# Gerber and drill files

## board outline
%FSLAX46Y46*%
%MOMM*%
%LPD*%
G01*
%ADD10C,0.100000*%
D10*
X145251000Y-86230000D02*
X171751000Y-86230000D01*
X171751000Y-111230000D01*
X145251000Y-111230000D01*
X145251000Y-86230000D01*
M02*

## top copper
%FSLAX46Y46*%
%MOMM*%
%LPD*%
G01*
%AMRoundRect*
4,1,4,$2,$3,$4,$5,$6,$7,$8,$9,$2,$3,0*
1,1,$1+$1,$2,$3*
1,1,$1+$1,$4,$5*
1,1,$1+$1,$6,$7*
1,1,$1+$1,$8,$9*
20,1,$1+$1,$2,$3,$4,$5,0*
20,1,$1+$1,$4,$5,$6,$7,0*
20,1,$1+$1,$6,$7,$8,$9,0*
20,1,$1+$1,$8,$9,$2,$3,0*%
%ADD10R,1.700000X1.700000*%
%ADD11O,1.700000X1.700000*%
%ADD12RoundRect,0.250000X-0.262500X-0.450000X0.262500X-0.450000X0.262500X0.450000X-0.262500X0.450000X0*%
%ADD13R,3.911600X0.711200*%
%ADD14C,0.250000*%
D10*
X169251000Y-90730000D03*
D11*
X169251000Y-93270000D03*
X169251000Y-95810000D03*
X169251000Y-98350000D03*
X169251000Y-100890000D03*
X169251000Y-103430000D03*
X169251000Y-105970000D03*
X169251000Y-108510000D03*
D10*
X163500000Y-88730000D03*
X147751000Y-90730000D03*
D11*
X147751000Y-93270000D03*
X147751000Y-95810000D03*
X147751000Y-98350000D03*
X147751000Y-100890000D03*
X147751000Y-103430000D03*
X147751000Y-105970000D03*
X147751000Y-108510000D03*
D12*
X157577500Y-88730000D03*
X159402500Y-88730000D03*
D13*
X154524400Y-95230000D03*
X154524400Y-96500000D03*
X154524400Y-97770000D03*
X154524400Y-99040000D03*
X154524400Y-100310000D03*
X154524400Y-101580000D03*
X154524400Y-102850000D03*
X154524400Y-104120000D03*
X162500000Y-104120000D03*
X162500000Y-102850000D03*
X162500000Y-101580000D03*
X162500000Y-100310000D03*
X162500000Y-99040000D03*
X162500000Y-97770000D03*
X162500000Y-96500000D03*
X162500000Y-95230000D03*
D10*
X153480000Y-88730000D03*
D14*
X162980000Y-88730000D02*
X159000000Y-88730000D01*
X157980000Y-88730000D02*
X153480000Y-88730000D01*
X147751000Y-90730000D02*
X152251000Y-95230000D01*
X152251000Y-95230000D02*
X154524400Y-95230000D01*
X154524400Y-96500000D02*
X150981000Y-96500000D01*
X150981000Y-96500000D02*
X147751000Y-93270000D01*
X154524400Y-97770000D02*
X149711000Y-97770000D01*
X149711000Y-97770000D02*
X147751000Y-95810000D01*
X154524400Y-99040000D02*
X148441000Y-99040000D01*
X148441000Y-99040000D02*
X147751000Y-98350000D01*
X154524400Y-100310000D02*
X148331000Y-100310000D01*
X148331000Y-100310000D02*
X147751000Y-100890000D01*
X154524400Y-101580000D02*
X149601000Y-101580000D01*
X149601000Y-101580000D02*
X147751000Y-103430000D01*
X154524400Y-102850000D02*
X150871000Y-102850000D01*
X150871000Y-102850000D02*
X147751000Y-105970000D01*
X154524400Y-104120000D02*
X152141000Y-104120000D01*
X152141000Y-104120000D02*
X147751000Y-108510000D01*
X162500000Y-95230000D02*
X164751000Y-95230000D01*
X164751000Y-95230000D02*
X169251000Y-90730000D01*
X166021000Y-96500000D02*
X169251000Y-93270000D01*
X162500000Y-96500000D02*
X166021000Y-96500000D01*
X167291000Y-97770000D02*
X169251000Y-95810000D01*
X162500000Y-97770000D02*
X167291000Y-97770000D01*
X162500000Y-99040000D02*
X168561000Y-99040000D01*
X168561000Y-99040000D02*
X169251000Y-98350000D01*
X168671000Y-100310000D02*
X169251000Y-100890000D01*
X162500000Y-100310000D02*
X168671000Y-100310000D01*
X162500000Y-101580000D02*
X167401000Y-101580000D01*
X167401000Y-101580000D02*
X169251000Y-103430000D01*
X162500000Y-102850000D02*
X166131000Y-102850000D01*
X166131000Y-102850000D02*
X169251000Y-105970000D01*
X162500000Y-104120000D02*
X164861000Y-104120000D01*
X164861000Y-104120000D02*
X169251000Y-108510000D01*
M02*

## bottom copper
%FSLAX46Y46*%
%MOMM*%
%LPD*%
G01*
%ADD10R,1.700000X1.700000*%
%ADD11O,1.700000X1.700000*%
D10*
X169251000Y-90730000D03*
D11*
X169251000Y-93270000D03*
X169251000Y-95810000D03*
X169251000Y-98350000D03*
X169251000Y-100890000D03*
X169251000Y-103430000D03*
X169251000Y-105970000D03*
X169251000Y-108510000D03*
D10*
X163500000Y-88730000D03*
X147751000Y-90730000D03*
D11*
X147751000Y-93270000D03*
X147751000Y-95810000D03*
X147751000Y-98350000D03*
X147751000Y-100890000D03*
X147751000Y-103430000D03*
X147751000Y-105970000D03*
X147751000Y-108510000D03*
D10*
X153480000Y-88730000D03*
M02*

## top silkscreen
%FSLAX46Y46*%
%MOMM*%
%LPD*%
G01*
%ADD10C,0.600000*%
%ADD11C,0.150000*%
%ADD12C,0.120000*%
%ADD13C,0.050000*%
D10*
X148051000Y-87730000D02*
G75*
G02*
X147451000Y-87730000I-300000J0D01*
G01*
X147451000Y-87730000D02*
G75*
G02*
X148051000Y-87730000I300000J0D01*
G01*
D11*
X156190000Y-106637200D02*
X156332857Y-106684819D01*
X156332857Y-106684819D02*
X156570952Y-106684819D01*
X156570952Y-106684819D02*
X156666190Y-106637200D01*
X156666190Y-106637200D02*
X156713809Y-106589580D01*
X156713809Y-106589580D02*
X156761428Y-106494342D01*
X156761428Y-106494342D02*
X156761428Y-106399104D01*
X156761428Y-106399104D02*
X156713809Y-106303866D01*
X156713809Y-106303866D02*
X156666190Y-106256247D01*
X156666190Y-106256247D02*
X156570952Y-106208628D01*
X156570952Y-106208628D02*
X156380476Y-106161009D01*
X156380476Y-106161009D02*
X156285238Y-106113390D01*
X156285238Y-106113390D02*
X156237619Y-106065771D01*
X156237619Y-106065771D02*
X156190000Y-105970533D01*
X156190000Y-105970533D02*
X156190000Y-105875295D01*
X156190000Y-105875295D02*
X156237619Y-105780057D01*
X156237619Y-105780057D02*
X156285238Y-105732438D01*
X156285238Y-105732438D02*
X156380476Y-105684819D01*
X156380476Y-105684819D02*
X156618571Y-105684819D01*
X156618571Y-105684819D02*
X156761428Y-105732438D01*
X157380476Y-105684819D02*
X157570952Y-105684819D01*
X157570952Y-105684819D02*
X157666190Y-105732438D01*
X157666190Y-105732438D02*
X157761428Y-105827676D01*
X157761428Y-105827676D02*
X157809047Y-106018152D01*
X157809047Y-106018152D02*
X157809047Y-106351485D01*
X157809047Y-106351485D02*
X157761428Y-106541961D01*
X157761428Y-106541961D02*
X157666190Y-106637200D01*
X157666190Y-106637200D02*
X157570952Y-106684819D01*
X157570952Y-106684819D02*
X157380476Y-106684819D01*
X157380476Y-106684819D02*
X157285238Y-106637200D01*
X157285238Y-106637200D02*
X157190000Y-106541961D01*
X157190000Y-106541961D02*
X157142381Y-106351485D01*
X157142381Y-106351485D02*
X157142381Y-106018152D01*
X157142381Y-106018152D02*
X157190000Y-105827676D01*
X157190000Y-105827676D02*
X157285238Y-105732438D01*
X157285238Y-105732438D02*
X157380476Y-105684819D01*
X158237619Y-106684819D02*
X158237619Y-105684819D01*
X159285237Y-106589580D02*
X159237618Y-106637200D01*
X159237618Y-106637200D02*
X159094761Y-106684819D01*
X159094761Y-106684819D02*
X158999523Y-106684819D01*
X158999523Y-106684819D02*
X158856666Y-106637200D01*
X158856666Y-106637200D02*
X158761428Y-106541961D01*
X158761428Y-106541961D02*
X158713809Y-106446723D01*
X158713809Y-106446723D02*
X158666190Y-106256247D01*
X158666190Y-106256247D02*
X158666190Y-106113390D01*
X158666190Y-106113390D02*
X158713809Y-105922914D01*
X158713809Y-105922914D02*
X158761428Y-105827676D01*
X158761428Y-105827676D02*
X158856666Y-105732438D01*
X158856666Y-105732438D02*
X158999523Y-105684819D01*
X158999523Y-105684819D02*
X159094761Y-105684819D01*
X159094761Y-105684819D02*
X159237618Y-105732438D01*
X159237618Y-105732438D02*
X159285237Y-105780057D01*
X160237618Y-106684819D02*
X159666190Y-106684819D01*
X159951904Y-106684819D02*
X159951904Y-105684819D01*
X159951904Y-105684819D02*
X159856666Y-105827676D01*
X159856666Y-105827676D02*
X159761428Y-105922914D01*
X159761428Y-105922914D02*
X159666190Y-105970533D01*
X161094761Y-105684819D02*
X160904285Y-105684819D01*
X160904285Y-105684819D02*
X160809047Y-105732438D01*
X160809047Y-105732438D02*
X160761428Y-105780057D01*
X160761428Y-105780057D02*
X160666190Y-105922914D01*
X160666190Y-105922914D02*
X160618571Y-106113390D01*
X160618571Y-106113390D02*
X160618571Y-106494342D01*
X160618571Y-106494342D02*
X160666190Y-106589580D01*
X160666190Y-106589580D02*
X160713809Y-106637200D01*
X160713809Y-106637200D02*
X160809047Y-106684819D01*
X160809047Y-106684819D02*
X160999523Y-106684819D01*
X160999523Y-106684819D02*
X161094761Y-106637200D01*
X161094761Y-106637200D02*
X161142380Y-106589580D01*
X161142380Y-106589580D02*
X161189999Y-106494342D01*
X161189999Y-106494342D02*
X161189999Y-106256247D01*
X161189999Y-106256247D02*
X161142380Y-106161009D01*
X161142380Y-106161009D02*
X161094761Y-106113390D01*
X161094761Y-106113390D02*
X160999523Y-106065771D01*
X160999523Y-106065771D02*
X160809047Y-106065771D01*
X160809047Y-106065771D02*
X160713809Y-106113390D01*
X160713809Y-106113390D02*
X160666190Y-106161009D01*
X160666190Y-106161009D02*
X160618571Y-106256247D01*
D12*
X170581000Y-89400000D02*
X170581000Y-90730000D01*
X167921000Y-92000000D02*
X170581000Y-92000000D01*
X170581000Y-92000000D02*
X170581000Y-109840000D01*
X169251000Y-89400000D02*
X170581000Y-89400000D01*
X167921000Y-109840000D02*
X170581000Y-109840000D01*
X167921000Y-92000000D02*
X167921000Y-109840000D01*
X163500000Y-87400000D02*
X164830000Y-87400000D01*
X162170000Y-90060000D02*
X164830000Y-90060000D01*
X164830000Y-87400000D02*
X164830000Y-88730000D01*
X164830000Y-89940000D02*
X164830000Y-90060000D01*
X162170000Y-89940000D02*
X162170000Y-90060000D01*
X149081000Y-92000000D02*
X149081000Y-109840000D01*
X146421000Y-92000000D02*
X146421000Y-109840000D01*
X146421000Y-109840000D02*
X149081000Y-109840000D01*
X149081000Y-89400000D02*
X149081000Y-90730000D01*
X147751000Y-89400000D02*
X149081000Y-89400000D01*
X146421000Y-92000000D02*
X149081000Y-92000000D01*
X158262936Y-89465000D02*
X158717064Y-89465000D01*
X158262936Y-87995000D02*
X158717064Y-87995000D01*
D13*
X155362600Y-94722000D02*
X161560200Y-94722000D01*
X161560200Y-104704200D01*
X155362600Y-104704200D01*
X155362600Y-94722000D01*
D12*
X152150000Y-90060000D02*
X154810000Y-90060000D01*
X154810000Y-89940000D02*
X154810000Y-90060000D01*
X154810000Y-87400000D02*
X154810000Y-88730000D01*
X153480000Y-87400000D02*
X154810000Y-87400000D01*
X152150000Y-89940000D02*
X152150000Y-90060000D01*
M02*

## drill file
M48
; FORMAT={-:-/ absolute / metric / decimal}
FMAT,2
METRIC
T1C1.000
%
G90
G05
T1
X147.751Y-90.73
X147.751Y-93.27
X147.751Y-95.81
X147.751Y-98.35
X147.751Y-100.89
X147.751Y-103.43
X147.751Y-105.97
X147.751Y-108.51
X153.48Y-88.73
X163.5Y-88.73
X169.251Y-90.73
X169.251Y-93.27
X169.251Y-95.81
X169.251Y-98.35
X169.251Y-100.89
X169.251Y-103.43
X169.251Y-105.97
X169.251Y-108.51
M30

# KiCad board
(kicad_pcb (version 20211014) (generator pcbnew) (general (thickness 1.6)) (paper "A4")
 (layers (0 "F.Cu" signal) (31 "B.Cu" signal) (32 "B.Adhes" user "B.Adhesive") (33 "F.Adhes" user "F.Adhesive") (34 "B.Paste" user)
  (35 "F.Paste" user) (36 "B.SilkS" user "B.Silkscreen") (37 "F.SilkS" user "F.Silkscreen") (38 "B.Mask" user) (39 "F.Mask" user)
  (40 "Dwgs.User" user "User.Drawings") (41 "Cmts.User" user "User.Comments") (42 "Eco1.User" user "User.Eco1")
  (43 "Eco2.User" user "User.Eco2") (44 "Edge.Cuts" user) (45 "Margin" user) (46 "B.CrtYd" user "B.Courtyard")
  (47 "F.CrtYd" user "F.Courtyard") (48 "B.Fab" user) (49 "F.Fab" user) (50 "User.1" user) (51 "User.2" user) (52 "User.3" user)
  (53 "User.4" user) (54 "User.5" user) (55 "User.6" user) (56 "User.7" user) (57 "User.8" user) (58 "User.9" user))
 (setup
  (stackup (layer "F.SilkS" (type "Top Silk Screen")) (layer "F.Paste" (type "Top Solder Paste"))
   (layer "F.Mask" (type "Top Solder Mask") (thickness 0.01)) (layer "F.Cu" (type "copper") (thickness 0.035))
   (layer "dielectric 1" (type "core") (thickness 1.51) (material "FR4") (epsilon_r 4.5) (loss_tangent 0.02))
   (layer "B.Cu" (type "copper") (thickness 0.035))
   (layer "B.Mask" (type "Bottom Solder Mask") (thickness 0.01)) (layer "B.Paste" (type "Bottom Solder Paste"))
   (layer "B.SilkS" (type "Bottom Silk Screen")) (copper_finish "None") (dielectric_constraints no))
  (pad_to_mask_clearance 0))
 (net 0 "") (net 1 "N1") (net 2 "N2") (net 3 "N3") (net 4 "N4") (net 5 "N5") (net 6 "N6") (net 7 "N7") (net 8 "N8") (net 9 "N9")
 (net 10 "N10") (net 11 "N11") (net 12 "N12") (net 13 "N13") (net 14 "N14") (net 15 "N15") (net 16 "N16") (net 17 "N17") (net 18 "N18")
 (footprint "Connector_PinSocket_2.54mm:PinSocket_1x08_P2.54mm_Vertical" (layer "F.Cu") (at 169.251 90.73)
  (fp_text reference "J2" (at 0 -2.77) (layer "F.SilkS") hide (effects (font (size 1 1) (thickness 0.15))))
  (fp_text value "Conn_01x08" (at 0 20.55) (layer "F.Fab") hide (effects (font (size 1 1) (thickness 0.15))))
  (fp_line (start 1.33 -1.33) (end 1.33 0) (layer "F.SilkS") (width 0.12))
  (fp_line (start -1.33 1.27) (end 1.33 1.27) (layer "F.SilkS") (width 0.12))
  (fp_line (start 1.33 1.27) (end 1.33 19.11) (layer "F.SilkS") (width 0.12))
  (fp_line (start 0 -1.33) (end 1.33 -1.33) (layer "F.SilkS") (width 0.12))
  (fp_line (start -1.33 19.11) (end 1.33 19.11) (layer "F.SilkS") (width 0.12))
  (fp_line (start -1.33 1.27) (end -1.33 19.11) (layer "F.SilkS") (width 0.12))
  (pad "1" thru_hole rect (at 0 0) (size 1.7 1.7) (drill 1) (layers *.Cu *.Mask) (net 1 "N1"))
  (pad "2" thru_hole oval (at 0 2.54) (size 1.7 1.7) (drill 1) (layers *.Cu *.Mask) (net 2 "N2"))
  (pad "3" thru_hole oval (at 0 5.08) (size 1.7 1.7) (drill 1) (layers *.Cu *.Mask) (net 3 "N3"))
  (pad "4" thru_hole oval (at 0 7.62) (size 1.7 1.7) (drill 1) (layers *.Cu *.Mask) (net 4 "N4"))
  (pad "5" thru_hole oval (at 0 10.16) (size 1.7 1.7) (drill 1) (layers *.Cu *.Mask) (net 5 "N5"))
  (pad "6" thru_hole oval (at 0 12.7) (size 1.7 1.7) (drill 1) (layers *.Cu *.Mask) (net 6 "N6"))
  (pad "7" thru_hole oval (at 0 15.24) (size 1.7 1.7) (drill 1) (layers *.Cu *.Mask) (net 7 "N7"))
  (pad "8" thru_hole oval (at 0 17.78) (size 1.7 1.7) (drill 1) (layers *.Cu *.Mask) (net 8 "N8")))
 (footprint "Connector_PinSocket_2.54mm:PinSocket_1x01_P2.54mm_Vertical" (layer "F.Cu") (at 163.5 88.73)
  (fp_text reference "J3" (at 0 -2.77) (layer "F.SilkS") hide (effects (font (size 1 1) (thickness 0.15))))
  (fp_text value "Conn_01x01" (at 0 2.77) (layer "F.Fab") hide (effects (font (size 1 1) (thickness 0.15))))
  (fp_line (start 0 -1.33) (end 1.33 -1.33) (layer "F.SilkS") (width 0.12))
  (fp_line (start -1.33 1.33) (end 1.33 1.33) (layer "F.SilkS") (width 0.12))
  (fp_line (start 1.33 -1.33) (end 1.33 0) (layer "F.SilkS") (width 0.12))
  (fp_line (start 1.33 1.21) (end 1.33 1.33) (layer "F.SilkS") (width 0.12))
  (fp_line (start -1.33 1.21) (end -1.33 1.33) (layer "F.SilkS") (width 0.12))
  (pad "1" thru_hole rect (at 0 0) (size 1.7 1.7) (drill 1) (layers *.Cu *.Mask) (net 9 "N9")))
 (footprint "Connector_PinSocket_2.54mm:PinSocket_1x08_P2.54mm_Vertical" (layer "F.Cu") (at 147.751 90.73)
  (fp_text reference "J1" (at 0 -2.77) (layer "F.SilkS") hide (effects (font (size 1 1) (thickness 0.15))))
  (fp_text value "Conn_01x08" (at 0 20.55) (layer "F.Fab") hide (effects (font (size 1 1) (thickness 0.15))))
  (fp_line (start 1.33 1.27) (end 1.33 19.11) (layer "F.SilkS") (width 0.12))
  (fp_line (start -1.33 1.27) (end -1.33 19.11) (layer "F.SilkS") (width 0.12))
  (fp_line (start -1.33 19.11) (end 1.33 19.11) (layer "F.SilkS") (width 0.12))
  (fp_line (start 1.33 -1.33) (end 1.33 0) (layer "F.SilkS") (width 0.12))
  (fp_line (start 0 -1.33) (end 1.33 -1.33) (layer "F.SilkS") (width 0.12))
  (fp_line (start -1.33 1.27) (end 1.33 1.27) (layer "F.SilkS") (width 0.12))
  (pad "1" thru_hole rect (at 0 0) (size 1.7 1.7) (drill 1) (layers *.Cu *.Mask) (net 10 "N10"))
  (pad "2" thru_hole oval (at 0 2.54) (size 1.7 1.7) (drill 1) (layers *.Cu *.Mask) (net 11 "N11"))
  (pad "3" thru_hole oval (at 0 5.08) (size 1.7 1.7) (drill 1) (layers *.Cu *.Mask) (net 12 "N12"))
  (pad "4" thru_hole oval (at 0 7.62) (size 1.7 1.7) (drill 1) (layers *.Cu *.Mask) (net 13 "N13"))
  (pad "5" thru_hole oval (at 0 10.16) (size 1.7 1.7) (drill 1) (layers *.Cu *.Mask) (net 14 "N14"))
  (pad "6" thru_hole oval (at 0 12.7) (size 1.7 1.7) (drill 1) (layers *.Cu *.Mask) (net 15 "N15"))
  (pad "7" thru_hole oval (at 0 15.24) (size 1.7 1.7) (drill 1) (layers *.Cu *.Mask) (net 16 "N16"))
  (pad "8" thru_hole oval (at 0 17.78) (size 1.7 1.7) (drill 1) (layers *.Cu *.Mask) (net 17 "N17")))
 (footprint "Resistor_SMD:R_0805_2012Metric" (layer "F.Cu") (at 158.49 88.73)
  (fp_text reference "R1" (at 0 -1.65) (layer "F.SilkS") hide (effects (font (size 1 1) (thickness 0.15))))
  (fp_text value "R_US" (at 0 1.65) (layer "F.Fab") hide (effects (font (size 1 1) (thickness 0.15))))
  (fp_line (start -0.227064 0.735) (end 0.227064 0.735) (layer "F.SilkS") (width 0.12))
  (fp_line (start -0.227064 -0.735) (end 0.227064 -0.735) (layer "F.SilkS") (width 0.12))
  (pad "1" smd roundrect (at -0.9125 0) (size 1.025 1.4) (layers "F.Cu" "F.Paste" "F.Mask") (roundrect_rratio 0.243902) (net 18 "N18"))
  (pad "2" smd roundrect (at 0.9125 0) (size 1.025 1.4) (layers "F.Cu" "F.Paste" "F.Mask") (roundrect_rratio 0.243902) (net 9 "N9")))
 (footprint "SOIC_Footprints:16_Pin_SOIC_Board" (layer "F.Cu") (at 158.69 99.548)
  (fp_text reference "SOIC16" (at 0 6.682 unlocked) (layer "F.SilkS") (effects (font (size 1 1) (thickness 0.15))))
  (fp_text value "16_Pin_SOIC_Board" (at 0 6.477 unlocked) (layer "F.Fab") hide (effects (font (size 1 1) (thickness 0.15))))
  (fp_rect (start -3.3274 -4.826) (end 2.8702 5.1562) (layer "F.SilkS") (width 0.05) (fill none))
  (pad "1" smd rect (at -4.1656 -4.318) (size 3.9116 0.7112) (layers "F.Cu" "F.Paste" "F.Mask") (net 10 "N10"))
  (pad "2" smd rect (at -4.1656 -3.048) (size 3.9116 0.7112) (layers "F.Cu" "F.Paste" "F.Mask") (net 11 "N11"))
  (pad "3" smd rect (at -4.1656 -1.778) (size 3.9116 0.7112) (layers "F.Cu" "F.Paste" "F.Mask") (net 12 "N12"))
  (pad "4" smd rect (at -4.1656 -0.508) (size 3.9116 0.7112) (layers "F.Cu" "F.Paste" "F.Mask") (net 13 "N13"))
  (pad "5" smd rect (at -4.1656 0.762) (size 3.9116 0.7112) (layers "F.Cu" "F.Paste" "F.Mask") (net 14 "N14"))
  (pad "6" smd rect (at -4.1656 2.032) (size 3.9116 0.7112) (layers "F.Cu" "F.Paste" "F.Mask") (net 15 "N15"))
  (pad "7" smd rect (at -4.1656 3.302) (size 3.9116 0.7112) (layers "F.Cu" "F.Paste" "F.Mask") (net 16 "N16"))
  (pad "8" smd rect (at -4.1656 4.572) (size 3.9116 0.7112) (layers "F.Cu" "F.Paste" "F.Mask") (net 17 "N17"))
  (pad "9" smd rect (at 3.81 4.572) (size 3.9116 0.7112) (layers "F.Cu" "F.Paste" "F.Mask") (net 8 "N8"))
  (pad "10" smd rect (at 3.81 3.302) (size 3.9116 0.7112) (layers "F.Cu" "F.Paste" "F.Mask") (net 7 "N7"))
  (pad "11" smd rect (at 3.81 2.032) (size 3.9116 0.7112) (layers "F.Cu" "F.Paste" "F.Mask") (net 6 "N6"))
  (pad "12" smd rect (at 3.81 0.762) (size 3.9116 0.7112) (layers "F.Cu" "F.Paste" "F.Mask") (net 5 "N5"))
  (pad "13" smd rect (at 3.81 -0.508) (size 3.9116 0.7112) (layers "F.Cu" "F.Paste" "F.Mask") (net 4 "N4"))
  (pad "14" smd rect (at 3.81 -1.778) (size 3.9116 0.7112) (layers "F.Cu" "F.Paste" "F.Mask") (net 3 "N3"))
  (pad "15" smd rect (at 3.81 -3.048) (size 3.9116 0.7112) (layers "F.Cu" "F.Paste" "F.Mask") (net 2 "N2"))
  (pad "16" smd rect (at 3.81 -4.318) (size 3.9116 0.7112) (layers "F.Cu" "F.Paste" "F.Mask") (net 1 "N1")))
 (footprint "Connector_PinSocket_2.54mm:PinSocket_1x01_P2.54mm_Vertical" (layer "F.Cu") (at 153.48 88.73)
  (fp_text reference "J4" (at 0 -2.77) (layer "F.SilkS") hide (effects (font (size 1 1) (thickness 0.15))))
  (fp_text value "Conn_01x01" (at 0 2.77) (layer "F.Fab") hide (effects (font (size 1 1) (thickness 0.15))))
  (fp_line (start -1.33 1.33) (end 1.33 1.33) (layer "F.SilkS") (width 0.12))
  (fp_line (start 1.33 1.21) (end 1.33 1.33) (layer "F.SilkS") (width 0.12))
  (fp_line (start 1.33 -1.33) (end 1.33 0) (layer "F.SilkS") (width 0.12))
  (fp_line (start 0 -1.33) (end 1.33 -1.33) (layer "F.SilkS") (width 0.12))
  (fp_line (start -1.33 1.21) (end -1.33 1.33) (layer "F.SilkS") (width 0.12))
  (pad "1" thru_hole rect (at 0 0) (size 1.7 1.7) (drill 1) (layers *.Cu *.Mask) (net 18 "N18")))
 (gr_circle (center 147.751 87.73) (end 148.251 87.73) (layer "F.SilkS") (width 0.2) (fill solid))
 (gr_rect (start 145.251 86.23) (end 171.751 111.23) (layer "Edge.Cuts") (width 0.1) (fill none))
 (segment (start 162.98 88.73) (end 159 88.73) (width 0.25) (layer "F.Cu") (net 9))
 (segment (start 157.98 88.73) (end 153.48 88.73) (width 0.25) (layer "F.Cu") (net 18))
 (segment (start 147.751 90.73) (end 152.251 95.23) (width 0.25) (layer "F.Cu") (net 10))
 (segment (start 152.251 95.23) (end 154.5244 95.23) (width 0.25) (layer "F.Cu") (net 10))
 (segment (start 154.5244 96.5) (end 150.981 96.5) (width 0.25) (layer "F.Cu") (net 11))
 (segment (start 150.981 96.5) (end 147.751 93.27) (width 0.25) (layer "F.Cu") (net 11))
 (segment (start 154.5244 97.77) (end 149.711 97.77) (width 0.25) (layer "F.Cu") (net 12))
 (segment (start 149.711 97.77) (end 147.751 95.81) (width 0.25) (layer "F.Cu") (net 12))
 (segment (start 154.5244 99.04) (end 148.441 99.04) (width 0.25) (layer "F.Cu") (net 13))
 (segment (start 148.441 99.04) (end 147.751 98.35) (width 0.25) (layer "F.Cu") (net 13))
 (segment (start 154.5244 100.31) (end 148.331 100.31) (width 0.25) (layer "F.Cu") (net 14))
 (segment (start 148.331 100.31) (end 147.751 100.89) (width 0.25) (layer "F.Cu") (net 14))
 (segment (start 154.5244 101.58) (end 149.601 101.58) (width 0.25) (layer "F.Cu") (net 15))
 (segment (start 149.601 101.58) (end 147.751 103.43) (width 0.25) (layer "F.Cu") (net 15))
 (segment (start 154.5244 102.85) (end 150.871 102.85) (width 0.25) (layer "F.Cu") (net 16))
 (segment (start 150.871 102.85) (end 147.751 105.97) (width 0.25) (layer "F.Cu") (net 16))
 (segment (start 154.5244 104.12) (end 152.141 104.12) (width 0.25) (layer "F.Cu") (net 17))
 (segment (start 152.141 104.12) (end 147.751 108.51) (width 0.25) (layer "F.Cu") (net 17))
 (segment (start 162.5 95.23) (end 164.751 95.23) (width 0.25) (layer "F.Cu") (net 1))
 (segment (start 164.751 95.23) (end 169.251 90.73) (width 0.25) (layer "F.Cu") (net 1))
 (segment (start 166.021 96.5) (end 169.251 93.27) (width 0.25) (layer "F.Cu") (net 2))
 (segment (start 162.5 96.5) (end 166.021 96.5) (width 0.25) (layer "F.Cu") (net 2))
 (segment (start 167.291 97.77) (end 169.251 95.81) (width 0.25) (layer "F.Cu") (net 3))
 (segment (start 162.5 97.77) (end 167.291 97.77) (width 0.25) (layer "F.Cu") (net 3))
 (segment (start 162.5 99.04) (end 168.561 99.04) (width 0.25) (layer "F.Cu") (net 4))
 (segment (start 168.561 99.04) (end 169.251 98.35) (width 0.25) (layer "F.Cu") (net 4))
 (segment (start 168.671 100.31) (end 169.251 100.89) (width 0.25) (layer "F.Cu") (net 5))
 (segment (start 162.5 100.31) (end 168.671 100.31) (width 0.25) (layer "F.Cu") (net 5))
 (segment (start 162.5 101.58) (end 167.401 101.58) (width 0.25) (layer "F.Cu") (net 6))
 (segment (start 167.401 101.58) (end 169.251 103.43) (width 0.25) (layer "F.Cu") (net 6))
 (segment (start 162.5 102.85) (end 166.131 102.85) (width 0.25) (layer "F.Cu") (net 7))
 (segment (start 166.131 102.85) (end 169.251 105.97) (width 0.25) (layer "F.Cu") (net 7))
 (segment (start 162.5 104.12) (end 164.861 104.12) (width 0.25) (layer "F.Cu") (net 8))
 (segment (start 164.861 104.12) (end 169.251 108.51) (width 0.25) (layer "F.Cu") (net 8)))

